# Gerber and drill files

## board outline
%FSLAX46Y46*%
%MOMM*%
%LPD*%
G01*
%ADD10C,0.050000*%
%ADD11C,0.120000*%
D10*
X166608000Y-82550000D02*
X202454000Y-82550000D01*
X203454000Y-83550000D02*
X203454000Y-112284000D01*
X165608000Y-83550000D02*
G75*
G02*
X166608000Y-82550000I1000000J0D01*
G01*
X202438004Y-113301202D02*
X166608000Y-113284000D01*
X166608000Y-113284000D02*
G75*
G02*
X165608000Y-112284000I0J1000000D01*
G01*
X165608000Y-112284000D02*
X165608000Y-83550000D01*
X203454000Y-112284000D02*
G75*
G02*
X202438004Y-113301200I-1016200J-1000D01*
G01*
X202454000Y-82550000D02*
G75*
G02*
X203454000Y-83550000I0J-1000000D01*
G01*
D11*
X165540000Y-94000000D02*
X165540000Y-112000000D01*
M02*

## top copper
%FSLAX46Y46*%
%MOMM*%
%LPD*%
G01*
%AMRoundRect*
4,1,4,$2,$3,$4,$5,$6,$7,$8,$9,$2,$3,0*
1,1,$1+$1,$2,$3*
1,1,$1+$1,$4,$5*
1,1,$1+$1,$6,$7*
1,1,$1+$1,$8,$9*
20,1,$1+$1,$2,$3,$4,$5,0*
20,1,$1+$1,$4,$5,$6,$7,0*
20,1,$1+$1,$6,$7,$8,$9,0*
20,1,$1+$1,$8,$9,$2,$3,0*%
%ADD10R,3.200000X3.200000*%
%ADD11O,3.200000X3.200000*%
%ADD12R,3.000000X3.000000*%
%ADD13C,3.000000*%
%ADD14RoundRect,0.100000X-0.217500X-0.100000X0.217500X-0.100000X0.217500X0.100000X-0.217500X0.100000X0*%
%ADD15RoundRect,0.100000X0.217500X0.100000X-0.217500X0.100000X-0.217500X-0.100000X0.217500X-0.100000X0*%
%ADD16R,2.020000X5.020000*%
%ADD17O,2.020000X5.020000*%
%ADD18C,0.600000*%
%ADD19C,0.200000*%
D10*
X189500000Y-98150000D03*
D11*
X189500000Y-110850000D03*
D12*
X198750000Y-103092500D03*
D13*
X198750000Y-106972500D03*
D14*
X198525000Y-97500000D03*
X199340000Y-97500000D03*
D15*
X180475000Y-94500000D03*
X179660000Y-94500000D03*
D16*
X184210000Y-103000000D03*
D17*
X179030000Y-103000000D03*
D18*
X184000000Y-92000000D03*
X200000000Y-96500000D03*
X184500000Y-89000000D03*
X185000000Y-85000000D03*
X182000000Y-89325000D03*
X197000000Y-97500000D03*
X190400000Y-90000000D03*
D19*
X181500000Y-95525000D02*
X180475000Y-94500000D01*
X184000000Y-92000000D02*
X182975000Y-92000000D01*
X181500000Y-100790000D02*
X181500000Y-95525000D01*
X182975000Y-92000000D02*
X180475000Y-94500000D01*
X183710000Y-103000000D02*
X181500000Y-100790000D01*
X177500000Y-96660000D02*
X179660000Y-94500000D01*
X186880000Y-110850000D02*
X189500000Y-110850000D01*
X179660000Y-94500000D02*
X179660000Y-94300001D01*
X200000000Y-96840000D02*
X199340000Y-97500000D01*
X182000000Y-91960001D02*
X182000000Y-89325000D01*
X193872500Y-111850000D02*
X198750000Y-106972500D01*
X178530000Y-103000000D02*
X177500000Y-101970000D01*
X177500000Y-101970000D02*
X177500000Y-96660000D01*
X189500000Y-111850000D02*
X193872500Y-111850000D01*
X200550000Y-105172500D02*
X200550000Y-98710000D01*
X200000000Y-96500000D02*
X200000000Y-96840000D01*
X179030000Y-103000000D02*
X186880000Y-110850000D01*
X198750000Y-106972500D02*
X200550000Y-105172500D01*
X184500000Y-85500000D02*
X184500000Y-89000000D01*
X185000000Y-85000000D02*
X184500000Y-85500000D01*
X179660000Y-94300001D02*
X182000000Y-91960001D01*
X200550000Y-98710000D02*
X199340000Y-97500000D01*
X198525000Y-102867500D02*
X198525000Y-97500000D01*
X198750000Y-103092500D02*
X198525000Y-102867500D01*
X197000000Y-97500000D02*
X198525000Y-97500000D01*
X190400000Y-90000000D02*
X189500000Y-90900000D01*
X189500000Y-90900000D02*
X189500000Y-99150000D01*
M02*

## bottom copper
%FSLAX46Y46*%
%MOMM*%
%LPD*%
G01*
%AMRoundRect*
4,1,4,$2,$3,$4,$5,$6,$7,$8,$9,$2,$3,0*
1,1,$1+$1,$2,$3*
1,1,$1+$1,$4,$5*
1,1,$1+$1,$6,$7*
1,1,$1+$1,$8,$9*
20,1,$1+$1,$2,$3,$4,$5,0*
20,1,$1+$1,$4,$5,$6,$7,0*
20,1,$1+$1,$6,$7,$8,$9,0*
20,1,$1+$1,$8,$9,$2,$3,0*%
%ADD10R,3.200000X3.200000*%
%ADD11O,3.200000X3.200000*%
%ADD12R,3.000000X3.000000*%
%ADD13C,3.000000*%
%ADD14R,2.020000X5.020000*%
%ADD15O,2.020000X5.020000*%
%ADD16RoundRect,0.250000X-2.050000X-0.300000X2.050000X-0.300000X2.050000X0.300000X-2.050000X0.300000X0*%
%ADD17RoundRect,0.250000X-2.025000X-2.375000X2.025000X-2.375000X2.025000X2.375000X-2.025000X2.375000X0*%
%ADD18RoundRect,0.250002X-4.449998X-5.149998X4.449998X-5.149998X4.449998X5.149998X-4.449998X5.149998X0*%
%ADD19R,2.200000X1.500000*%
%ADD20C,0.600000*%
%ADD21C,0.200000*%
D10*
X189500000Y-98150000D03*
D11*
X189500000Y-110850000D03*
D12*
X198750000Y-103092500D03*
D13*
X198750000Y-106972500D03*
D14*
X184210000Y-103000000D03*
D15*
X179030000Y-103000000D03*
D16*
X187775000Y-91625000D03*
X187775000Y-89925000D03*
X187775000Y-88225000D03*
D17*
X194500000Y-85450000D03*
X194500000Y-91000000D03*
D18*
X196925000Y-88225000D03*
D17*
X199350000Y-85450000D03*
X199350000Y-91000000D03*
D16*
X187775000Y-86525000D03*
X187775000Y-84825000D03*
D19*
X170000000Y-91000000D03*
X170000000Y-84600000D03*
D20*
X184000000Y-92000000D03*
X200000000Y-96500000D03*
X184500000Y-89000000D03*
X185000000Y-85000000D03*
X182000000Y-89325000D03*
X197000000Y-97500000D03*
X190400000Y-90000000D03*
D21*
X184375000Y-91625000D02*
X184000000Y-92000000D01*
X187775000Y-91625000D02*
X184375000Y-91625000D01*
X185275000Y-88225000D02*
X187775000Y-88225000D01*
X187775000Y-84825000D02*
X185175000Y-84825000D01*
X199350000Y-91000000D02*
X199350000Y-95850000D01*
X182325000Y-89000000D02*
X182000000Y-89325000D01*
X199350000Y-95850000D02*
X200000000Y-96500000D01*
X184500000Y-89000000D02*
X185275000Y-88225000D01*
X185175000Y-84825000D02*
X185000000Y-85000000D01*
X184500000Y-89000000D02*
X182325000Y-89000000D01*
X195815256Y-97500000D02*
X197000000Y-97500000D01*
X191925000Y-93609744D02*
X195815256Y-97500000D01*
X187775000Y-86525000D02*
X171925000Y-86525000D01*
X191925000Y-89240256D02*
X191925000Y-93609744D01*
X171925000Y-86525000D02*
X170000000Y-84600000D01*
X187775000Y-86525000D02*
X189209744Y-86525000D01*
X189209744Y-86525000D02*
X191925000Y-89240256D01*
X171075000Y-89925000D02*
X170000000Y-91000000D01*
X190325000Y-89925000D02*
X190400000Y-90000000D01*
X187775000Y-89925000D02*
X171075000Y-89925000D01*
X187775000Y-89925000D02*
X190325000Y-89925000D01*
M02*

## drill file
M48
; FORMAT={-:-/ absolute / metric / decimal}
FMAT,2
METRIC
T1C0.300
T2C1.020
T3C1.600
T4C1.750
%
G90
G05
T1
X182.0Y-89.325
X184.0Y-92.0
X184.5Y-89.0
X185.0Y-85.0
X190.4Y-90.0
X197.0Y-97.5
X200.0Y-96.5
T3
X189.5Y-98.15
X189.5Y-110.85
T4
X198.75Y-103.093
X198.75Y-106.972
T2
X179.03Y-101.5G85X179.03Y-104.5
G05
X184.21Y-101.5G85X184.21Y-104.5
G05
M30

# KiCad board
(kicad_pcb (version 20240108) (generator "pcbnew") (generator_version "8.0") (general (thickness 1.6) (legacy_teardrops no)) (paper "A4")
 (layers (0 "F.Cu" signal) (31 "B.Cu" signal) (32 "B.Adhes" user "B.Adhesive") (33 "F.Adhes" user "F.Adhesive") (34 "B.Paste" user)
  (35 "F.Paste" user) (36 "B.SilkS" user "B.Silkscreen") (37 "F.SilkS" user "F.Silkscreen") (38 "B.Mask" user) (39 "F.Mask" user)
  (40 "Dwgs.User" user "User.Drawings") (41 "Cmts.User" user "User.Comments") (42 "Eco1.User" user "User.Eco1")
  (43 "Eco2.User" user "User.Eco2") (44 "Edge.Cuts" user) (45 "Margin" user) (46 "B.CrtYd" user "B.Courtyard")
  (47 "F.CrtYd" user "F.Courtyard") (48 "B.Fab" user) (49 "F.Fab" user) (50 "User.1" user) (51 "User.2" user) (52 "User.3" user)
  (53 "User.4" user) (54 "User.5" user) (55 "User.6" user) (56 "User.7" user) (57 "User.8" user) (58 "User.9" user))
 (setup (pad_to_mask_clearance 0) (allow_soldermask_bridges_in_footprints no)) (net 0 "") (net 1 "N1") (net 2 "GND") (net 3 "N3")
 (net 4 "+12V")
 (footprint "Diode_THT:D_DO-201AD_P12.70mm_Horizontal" (layer "F.Cu") (at 189.5 98.15 -90)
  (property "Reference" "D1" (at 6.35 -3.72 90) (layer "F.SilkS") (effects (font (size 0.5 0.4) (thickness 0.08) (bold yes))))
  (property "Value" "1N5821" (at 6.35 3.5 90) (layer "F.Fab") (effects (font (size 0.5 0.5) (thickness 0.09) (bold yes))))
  (pad "1" thru_hole rect (at 0 0 270) (size 3.2 3.2) (drill 1.6) (layers "*.Cu" "*.Mask") (remove_unused_layers no) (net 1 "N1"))
  (pad "2" thru_hole oval (at 12.7 0 270) (size 3.2 3.2) (drill 1.6) (layers "*.Cu" "*.Mask") (remove_unused_layers no) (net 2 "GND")))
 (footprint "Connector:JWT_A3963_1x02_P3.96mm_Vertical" (layer "F.Cu") (at 198.75 103.0925 -90)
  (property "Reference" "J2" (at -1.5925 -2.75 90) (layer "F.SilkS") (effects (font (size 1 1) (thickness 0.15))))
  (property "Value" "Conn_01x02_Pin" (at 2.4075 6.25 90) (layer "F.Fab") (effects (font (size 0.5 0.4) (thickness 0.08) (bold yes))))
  (pad "1" thru_hole rect (at 0 0 270) (size 3 3) (drill 1.75) (layers "*.Cu" "*.Mask") (remove_unused_layers no) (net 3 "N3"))
  (pad "2" thru_hole circle (at 3.88 0 270) (size 3 3) (drill 1.75) (layers "*.Cu" "*.Mask") (remove_unused_layers no) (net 2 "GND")))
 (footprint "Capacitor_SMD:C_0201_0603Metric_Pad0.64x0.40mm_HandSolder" (layer "F.Cu") (at 198.9325 97.5)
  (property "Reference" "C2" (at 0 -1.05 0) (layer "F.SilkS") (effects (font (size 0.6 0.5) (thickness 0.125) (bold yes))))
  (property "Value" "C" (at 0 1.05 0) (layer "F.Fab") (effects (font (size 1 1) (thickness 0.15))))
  (pad "" smd roundrect (at -0.4325 0) (size 0.458 0.36) (layers "F.Paste") (roundrect_rratio 0.25))
  (pad "" smd roundrect (at 0.4325 0) (size 0.458 0.36) (layers "F.Paste") (roundrect_rratio 0.25))
  (pad "1" smd roundrect (at -0.4075 0) (size 0.635 0.4) (layers "F.Cu" "F.Mask") (roundrect_rratio 0.25) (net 3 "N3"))
  (pad "2" smd roundrect (at 0.4075 0) (size 0.635 0.4) (layers "F.Cu" "F.Mask") (roundrect_rratio 0.25) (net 2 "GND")))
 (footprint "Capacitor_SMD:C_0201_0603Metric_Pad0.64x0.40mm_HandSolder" (layer "F.Cu") (at 180.0675 94.5 180)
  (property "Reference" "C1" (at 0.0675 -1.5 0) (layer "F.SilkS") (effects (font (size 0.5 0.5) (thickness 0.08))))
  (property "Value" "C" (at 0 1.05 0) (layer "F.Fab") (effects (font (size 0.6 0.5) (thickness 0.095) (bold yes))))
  (pad "" smd roundrect (at -0.4325 0 180) (size 0.458 0.36) (layers "F.Paste") (roundrect_rratio 0.25))
  (pad "" smd roundrect (at 0.4325 0 180) (size 0.458 0.36) (layers "F.Paste") (roundrect_rratio 0.25))
  (pad "1" smd roundrect (at -0.4075 0 180) (size 0.635 0.4) (layers "F.Cu" "F.Mask") (roundrect_rratio 0.25) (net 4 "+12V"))
  (pad "2" smd roundrect (at 0.4075 0 180) (size 0.635 0.4) (layers "F.Cu" "F.Mask") (roundrect_rratio 0.25) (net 2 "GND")))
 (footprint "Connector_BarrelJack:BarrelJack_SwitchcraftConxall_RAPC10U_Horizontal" (layer "F.Cu") (at 184.21 103)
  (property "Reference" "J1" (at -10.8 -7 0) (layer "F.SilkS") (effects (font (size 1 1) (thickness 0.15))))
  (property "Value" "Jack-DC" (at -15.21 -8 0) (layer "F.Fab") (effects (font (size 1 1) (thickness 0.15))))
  (fp_line (start -18.67 -9) (end -18.67 9) (stroke (width 0.12) (type solid)) (layer "Edge.Cuts"))
  (pad "1" thru_hole rect (at 0 0) (size 2.02 5.02) (drill oval 1.02 4.02) (layers "*.Cu" "*.Mask") (remove_unused_layers no) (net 4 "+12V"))
  (pad "2" thru_hole oval (at -5.18 0) (size 2.02 5.02) (drill oval 1.02 4.02) (layers "*.Cu" "*.Mask") (remove_unused_layers no)
   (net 2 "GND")))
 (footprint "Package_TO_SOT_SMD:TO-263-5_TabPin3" (layer "B.Cu") (at 195.425 88.225)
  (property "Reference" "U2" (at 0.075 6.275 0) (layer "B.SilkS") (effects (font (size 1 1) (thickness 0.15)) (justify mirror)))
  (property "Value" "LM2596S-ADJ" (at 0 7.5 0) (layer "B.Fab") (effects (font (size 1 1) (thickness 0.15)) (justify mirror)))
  (pad "1" smd roundrect (at -7.65 3.4) (size 4.6 1.1) (layers "B.Cu" "B.Paste" "B.Mask") (roundrect_rratio 0.227273) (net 4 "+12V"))
  (pad "2" smd roundrect (at -7.65 1.7) (size 4.6 1.1) (layers "B.Cu" "B.Paste" "B.Mask") (roundrect_rratio 0.227273) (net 1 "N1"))
  (pad "3" smd roundrect (at -7.65 0) (size 4.6 1.1) (layers "B.Cu" "B.Paste" "B.Mask") (roundrect_rratio 0.227273) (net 2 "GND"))
  (pad "3" smd roundrect (at -0.925 -2.775) (size 4.55 5.25) (layers "B.Cu" "B.Paste") (roundrect_rratio 0.054945) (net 2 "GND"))
  (pad "3" smd roundrect (at -0.925 2.775) (size 4.55 5.25) (layers "B.Cu" "B.Paste") (roundrect_rratio 0.054945) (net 2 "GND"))
  (pad "3" smd roundrect (at 1.5 0) (size 9.4 10.8) (layers "B.Cu" "B.Mask") (roundrect_rratio 0.026596) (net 2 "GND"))
  (pad "3" smd roundrect (at 3.925 -2.775) (size 4.55 5.25) (layers "B.Cu" "B.Paste") (roundrect_rratio 0.054945) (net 2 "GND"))
  (pad "3" smd roundrect (at 3.925 2.775) (size 4.55 5.25) (layers "B.Cu" "B.Paste") (roundrect_rratio 0.054945) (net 2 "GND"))
  (pad "4" smd roundrect (at -7.65 -1.7) (size 4.6 1.1) (layers "B.Cu" "B.Paste" "B.Mask") (roundrect_rratio 0.227273) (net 3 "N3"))
  (pad "5" smd roundrect (at -7.65 -3.4) (size 4.6 1.1) (layers "B.Cu" "B.Paste" "B.Mask") (roundrect_rratio 0.227273) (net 2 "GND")))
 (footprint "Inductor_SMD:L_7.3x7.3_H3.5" (layer "B.Cu") (at 170 87.8 90)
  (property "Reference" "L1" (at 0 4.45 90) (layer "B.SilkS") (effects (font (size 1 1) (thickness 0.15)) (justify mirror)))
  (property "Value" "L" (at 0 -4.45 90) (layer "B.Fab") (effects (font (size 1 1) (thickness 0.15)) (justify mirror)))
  (pad "1" smd rect (at -3.2 0 90) (size 1.5 2.2) (layers "B.Cu" "B.Paste" "B.Mask") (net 1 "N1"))
  (pad "2" smd rect (at 3.2 0 90) (size 1.5 2.2) (layers "B.Cu" "B.Paste" "B.Mask") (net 3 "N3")))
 (gr_line (start 166.608 82.55) (end 202.454 82.55) (stroke (width 0.05) (type default)) (layer "Edge.Cuts"))
 (gr_line (start 203.454 83.55) (end 203.454 112.284) (stroke (width 0.05) (type default)) (layer "Edge.Cuts"))
 (gr_arc (start 165.608 83.55) (mid 165.900893 82.842893) (end 166.608 82.55) (stroke (width 0.05) (type default)) (layer "Edge.Cuts"))
 (gr_line (start 202.438004 113.301202) (end 166.608 113.284) (stroke (width 0.05) (type default)) (layer "Edge.Cuts"))
 (gr_arc (start 166.608 113.284) (mid 165.900893 112.991107) (end 165.608 112.284) (stroke (width 0.05) (type default)) (layer "Edge.Cuts"))
 (gr_line (start 165.608 112.284) (end 165.608 83.55) (stroke (width 0.05) (type default)) (layer "Edge.Cuts"))
 (gr_arc (start 203.454 112.284) (mid 203.156776 113.003126) (end 202.438004 113.301202) (stroke (width 0.05) (type default))
  (layer "Edge.Cuts"))
 (gr_arc (start 202.454 82.55) (mid 203.161107 82.842893) (end 203.454 83.55) (stroke (width 0.05) (type default)) (layer "Edge.Cuts"))
 (segment (start 181.5 95.525) (end 180.475 94.5) (width 0.2) (layer "F.Cu") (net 4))
 (segment (start 184 92) (end 182.975 92) (width 0.2) (layer "F.Cu") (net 4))
 (segment (start 181.5 100.79) (end 181.5 95.525) (width 0.2) (layer "F.Cu") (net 4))
 (segment (start 182.975 92) (end 180.475 94.5) (width 0.2) (layer "F.Cu") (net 4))
 (segment (start 183.71 103) (end 181.5 100.79) (width 0.2) (layer "F.Cu") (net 4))
 (via (at 184 92) (size 0.6) (drill 0.3) (layers "F.Cu" "B.Cu") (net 4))
 (segment (start 184.375 91.625) (end 184 92) (width 0.2) (layer "B.Cu") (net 4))
 (segment (start 187.775 91.625) (end 184.375 91.625) (width 0.2) (layer "B.Cu") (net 4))
 (segment (start 177.5 96.66) (end 179.66 94.5) (width 0.2) (layer "F.Cu") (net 2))
 (segment (start 186.88 110.85) (end 189.5 110.85) (width 0.2) (layer "F.Cu") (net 2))
 (segment (start 179.66 94.5) (end 179.66 94.300001) (width 0.2) (layer "F.Cu") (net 2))
 (segment (start 200 96.84) (end 199.34 97.5) (width 0.2) (layer "F.Cu") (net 2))
 (segment (start 182 91.960001) (end 182 89.325) (width 0.2) (layer "F.Cu") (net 2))
 (segment (start 193.8725 111.85) (end 198.75 106.9725) (width 0.2) (layer "F.Cu") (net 2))
 (segment (start 178.53 103) (end 177.5 101.97) (width 0.2) (layer "F.Cu") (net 2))
 (segment (start 177.5 101.97) (end 177.5 96.66) (width 0.2) (layer "F.Cu") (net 2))
 (segment (start 189.5 111.85) (end 193.8725 111.85) (width 0.2) (layer "F.Cu") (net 2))
 (segment (start 200.55 105.1725) (end 200.55 98.71) (width 0.2) (layer "F.Cu") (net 2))
 (segment (start 200 96.5) (end 200 96.84) (width 0.2) (layer "F.Cu") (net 2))
 (segment (start 179.03 103) (end 186.88 110.85) (width 0.2) (layer "F.Cu") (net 2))
 (segment (start 198.75 106.9725) (end 200.55 105.1725) (width 0.2) (layer "F.Cu") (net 2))
 (segment (start 184.5 85.5) (end 184.5 89) (width 0.2) (layer "F.Cu") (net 2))
 (segment (start 185 85) (end 184.5 85.5) (width 0.2) (layer "F.Cu") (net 2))
 (segment (start 179.66 94.300001) (end 182 91.960001) (width 0.2) (layer "F.Cu") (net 2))
 (segment (start 200.55 98.71) (end 199.34 97.5) (width 0.2) (layer "F.Cu") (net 2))
 (via (at 200 96.5) (size 0.6) (drill 0.3) (layers "F.Cu" "B.Cu") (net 2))
 (via (at 184.5 89) (size 0.6) (drill 0.3) (layers "F.Cu" "B.Cu") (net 2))
 (via (at 185 85) (size 0.6) (drill 0.3) (layers "F.Cu" "B.Cu") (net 2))
 (via (at 182 89.325) (size 0.6) (drill 0.3) (layers "F.Cu" "B.Cu") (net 2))
 (segment (start 185.275 88.225) (end 187.775 88.225) (width 0.2) (layer "B.Cu") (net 2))
 (segment (start 187.775 84.825) (end 185.175 84.825) (width 0.2) (layer "B.Cu") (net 2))
 (segment (start 199.35 91) (end 199.35 95.85) (width 0.2) (layer "B.Cu") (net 2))
 (segment (start 182.325 89) (end 182 89.325) (width 0.2) (layer "B.Cu") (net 2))
 (segment (start 199.35 95.85) (end 200 96.5) (width 0.2) (layer "B.Cu") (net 2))
 (segment (start 184.5 89) (end 185.275 88.225) (width 0.2) (layer "B.Cu") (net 2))
 (segment (start 185.175 84.825) (end 185 85) (width 0.2) (layer "B.Cu") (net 2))
 (segment (start 184.5 89) (end 182.325 89) (width 0.2) (layer "B.Cu") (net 2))
 (segment (start 198.525 102.8675) (end 198.525 97.5) (width 0.2) (layer "F.Cu") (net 3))
 (segment (start 198.75 103.0925) (end 198.525 102.8675) (width 0.2) (layer "F.Cu") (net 3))
 (segment (start 197 97.5) (end 198.525 97.5) (width 0.2) (layer "F.Cu") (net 3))
 (via (at 197 97.5) (size 0.6) (drill 0.3) (layers "F.Cu" "B.Cu") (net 3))
 (segment (start 195.815256 97.5) (end 197 97.5) (width 0.2) (layer "B.Cu") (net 3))
 (segment (start 191.925 93.609744) (end 195.815256 97.5) (width 0.2) (layer "B.Cu") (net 3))
 (segment (start 187.775 86.525) (end 171.925 86.525) (width 0.2) (layer "B.Cu") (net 3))
 (segment (start 191.925 89.240256) (end 191.925 93.609744) (width 0.2) (layer "B.Cu") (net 3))
 (segment (start 171.925 86.525) (end 170 84.6) (width 0.2) (layer "B.Cu") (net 3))
 (segment (start 187.775 86.525) (end 189.209744 86.525) (width 0.2) (layer "B.Cu") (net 3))
 (segment (start 189.209744 86.525) (end 191.925 89.240256) (width 0.2) (layer "B.Cu") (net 3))
 (segment (start 190.4 90) (end 189.5 90.9) (width 0.2) (layer "F.Cu") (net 1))
 (segment (start 189.5 90.9) (end 189.5 99.15) (width 0.2) (layer "F.Cu") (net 1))
 (via (at 190.4 90) (size 0.6) (drill 0.3) (layers "F.Cu" "B.Cu") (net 1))
 (segment (start 171.075 89.925) (end 170 91) (width 0.2) (layer "B.Cu") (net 1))
 (segment (start 190.325 89.925) (end 190.4 90) (width 0.2) (layer "B.Cu") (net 1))
 (segment (start 187.775 89.925) (end 171.075 89.925) (width 0.2) (layer "B.Cu") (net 1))
 (segment (start 187.775 89.925) (end 190.325 89.925) (width 0.2) (layer "B.Cu") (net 1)))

